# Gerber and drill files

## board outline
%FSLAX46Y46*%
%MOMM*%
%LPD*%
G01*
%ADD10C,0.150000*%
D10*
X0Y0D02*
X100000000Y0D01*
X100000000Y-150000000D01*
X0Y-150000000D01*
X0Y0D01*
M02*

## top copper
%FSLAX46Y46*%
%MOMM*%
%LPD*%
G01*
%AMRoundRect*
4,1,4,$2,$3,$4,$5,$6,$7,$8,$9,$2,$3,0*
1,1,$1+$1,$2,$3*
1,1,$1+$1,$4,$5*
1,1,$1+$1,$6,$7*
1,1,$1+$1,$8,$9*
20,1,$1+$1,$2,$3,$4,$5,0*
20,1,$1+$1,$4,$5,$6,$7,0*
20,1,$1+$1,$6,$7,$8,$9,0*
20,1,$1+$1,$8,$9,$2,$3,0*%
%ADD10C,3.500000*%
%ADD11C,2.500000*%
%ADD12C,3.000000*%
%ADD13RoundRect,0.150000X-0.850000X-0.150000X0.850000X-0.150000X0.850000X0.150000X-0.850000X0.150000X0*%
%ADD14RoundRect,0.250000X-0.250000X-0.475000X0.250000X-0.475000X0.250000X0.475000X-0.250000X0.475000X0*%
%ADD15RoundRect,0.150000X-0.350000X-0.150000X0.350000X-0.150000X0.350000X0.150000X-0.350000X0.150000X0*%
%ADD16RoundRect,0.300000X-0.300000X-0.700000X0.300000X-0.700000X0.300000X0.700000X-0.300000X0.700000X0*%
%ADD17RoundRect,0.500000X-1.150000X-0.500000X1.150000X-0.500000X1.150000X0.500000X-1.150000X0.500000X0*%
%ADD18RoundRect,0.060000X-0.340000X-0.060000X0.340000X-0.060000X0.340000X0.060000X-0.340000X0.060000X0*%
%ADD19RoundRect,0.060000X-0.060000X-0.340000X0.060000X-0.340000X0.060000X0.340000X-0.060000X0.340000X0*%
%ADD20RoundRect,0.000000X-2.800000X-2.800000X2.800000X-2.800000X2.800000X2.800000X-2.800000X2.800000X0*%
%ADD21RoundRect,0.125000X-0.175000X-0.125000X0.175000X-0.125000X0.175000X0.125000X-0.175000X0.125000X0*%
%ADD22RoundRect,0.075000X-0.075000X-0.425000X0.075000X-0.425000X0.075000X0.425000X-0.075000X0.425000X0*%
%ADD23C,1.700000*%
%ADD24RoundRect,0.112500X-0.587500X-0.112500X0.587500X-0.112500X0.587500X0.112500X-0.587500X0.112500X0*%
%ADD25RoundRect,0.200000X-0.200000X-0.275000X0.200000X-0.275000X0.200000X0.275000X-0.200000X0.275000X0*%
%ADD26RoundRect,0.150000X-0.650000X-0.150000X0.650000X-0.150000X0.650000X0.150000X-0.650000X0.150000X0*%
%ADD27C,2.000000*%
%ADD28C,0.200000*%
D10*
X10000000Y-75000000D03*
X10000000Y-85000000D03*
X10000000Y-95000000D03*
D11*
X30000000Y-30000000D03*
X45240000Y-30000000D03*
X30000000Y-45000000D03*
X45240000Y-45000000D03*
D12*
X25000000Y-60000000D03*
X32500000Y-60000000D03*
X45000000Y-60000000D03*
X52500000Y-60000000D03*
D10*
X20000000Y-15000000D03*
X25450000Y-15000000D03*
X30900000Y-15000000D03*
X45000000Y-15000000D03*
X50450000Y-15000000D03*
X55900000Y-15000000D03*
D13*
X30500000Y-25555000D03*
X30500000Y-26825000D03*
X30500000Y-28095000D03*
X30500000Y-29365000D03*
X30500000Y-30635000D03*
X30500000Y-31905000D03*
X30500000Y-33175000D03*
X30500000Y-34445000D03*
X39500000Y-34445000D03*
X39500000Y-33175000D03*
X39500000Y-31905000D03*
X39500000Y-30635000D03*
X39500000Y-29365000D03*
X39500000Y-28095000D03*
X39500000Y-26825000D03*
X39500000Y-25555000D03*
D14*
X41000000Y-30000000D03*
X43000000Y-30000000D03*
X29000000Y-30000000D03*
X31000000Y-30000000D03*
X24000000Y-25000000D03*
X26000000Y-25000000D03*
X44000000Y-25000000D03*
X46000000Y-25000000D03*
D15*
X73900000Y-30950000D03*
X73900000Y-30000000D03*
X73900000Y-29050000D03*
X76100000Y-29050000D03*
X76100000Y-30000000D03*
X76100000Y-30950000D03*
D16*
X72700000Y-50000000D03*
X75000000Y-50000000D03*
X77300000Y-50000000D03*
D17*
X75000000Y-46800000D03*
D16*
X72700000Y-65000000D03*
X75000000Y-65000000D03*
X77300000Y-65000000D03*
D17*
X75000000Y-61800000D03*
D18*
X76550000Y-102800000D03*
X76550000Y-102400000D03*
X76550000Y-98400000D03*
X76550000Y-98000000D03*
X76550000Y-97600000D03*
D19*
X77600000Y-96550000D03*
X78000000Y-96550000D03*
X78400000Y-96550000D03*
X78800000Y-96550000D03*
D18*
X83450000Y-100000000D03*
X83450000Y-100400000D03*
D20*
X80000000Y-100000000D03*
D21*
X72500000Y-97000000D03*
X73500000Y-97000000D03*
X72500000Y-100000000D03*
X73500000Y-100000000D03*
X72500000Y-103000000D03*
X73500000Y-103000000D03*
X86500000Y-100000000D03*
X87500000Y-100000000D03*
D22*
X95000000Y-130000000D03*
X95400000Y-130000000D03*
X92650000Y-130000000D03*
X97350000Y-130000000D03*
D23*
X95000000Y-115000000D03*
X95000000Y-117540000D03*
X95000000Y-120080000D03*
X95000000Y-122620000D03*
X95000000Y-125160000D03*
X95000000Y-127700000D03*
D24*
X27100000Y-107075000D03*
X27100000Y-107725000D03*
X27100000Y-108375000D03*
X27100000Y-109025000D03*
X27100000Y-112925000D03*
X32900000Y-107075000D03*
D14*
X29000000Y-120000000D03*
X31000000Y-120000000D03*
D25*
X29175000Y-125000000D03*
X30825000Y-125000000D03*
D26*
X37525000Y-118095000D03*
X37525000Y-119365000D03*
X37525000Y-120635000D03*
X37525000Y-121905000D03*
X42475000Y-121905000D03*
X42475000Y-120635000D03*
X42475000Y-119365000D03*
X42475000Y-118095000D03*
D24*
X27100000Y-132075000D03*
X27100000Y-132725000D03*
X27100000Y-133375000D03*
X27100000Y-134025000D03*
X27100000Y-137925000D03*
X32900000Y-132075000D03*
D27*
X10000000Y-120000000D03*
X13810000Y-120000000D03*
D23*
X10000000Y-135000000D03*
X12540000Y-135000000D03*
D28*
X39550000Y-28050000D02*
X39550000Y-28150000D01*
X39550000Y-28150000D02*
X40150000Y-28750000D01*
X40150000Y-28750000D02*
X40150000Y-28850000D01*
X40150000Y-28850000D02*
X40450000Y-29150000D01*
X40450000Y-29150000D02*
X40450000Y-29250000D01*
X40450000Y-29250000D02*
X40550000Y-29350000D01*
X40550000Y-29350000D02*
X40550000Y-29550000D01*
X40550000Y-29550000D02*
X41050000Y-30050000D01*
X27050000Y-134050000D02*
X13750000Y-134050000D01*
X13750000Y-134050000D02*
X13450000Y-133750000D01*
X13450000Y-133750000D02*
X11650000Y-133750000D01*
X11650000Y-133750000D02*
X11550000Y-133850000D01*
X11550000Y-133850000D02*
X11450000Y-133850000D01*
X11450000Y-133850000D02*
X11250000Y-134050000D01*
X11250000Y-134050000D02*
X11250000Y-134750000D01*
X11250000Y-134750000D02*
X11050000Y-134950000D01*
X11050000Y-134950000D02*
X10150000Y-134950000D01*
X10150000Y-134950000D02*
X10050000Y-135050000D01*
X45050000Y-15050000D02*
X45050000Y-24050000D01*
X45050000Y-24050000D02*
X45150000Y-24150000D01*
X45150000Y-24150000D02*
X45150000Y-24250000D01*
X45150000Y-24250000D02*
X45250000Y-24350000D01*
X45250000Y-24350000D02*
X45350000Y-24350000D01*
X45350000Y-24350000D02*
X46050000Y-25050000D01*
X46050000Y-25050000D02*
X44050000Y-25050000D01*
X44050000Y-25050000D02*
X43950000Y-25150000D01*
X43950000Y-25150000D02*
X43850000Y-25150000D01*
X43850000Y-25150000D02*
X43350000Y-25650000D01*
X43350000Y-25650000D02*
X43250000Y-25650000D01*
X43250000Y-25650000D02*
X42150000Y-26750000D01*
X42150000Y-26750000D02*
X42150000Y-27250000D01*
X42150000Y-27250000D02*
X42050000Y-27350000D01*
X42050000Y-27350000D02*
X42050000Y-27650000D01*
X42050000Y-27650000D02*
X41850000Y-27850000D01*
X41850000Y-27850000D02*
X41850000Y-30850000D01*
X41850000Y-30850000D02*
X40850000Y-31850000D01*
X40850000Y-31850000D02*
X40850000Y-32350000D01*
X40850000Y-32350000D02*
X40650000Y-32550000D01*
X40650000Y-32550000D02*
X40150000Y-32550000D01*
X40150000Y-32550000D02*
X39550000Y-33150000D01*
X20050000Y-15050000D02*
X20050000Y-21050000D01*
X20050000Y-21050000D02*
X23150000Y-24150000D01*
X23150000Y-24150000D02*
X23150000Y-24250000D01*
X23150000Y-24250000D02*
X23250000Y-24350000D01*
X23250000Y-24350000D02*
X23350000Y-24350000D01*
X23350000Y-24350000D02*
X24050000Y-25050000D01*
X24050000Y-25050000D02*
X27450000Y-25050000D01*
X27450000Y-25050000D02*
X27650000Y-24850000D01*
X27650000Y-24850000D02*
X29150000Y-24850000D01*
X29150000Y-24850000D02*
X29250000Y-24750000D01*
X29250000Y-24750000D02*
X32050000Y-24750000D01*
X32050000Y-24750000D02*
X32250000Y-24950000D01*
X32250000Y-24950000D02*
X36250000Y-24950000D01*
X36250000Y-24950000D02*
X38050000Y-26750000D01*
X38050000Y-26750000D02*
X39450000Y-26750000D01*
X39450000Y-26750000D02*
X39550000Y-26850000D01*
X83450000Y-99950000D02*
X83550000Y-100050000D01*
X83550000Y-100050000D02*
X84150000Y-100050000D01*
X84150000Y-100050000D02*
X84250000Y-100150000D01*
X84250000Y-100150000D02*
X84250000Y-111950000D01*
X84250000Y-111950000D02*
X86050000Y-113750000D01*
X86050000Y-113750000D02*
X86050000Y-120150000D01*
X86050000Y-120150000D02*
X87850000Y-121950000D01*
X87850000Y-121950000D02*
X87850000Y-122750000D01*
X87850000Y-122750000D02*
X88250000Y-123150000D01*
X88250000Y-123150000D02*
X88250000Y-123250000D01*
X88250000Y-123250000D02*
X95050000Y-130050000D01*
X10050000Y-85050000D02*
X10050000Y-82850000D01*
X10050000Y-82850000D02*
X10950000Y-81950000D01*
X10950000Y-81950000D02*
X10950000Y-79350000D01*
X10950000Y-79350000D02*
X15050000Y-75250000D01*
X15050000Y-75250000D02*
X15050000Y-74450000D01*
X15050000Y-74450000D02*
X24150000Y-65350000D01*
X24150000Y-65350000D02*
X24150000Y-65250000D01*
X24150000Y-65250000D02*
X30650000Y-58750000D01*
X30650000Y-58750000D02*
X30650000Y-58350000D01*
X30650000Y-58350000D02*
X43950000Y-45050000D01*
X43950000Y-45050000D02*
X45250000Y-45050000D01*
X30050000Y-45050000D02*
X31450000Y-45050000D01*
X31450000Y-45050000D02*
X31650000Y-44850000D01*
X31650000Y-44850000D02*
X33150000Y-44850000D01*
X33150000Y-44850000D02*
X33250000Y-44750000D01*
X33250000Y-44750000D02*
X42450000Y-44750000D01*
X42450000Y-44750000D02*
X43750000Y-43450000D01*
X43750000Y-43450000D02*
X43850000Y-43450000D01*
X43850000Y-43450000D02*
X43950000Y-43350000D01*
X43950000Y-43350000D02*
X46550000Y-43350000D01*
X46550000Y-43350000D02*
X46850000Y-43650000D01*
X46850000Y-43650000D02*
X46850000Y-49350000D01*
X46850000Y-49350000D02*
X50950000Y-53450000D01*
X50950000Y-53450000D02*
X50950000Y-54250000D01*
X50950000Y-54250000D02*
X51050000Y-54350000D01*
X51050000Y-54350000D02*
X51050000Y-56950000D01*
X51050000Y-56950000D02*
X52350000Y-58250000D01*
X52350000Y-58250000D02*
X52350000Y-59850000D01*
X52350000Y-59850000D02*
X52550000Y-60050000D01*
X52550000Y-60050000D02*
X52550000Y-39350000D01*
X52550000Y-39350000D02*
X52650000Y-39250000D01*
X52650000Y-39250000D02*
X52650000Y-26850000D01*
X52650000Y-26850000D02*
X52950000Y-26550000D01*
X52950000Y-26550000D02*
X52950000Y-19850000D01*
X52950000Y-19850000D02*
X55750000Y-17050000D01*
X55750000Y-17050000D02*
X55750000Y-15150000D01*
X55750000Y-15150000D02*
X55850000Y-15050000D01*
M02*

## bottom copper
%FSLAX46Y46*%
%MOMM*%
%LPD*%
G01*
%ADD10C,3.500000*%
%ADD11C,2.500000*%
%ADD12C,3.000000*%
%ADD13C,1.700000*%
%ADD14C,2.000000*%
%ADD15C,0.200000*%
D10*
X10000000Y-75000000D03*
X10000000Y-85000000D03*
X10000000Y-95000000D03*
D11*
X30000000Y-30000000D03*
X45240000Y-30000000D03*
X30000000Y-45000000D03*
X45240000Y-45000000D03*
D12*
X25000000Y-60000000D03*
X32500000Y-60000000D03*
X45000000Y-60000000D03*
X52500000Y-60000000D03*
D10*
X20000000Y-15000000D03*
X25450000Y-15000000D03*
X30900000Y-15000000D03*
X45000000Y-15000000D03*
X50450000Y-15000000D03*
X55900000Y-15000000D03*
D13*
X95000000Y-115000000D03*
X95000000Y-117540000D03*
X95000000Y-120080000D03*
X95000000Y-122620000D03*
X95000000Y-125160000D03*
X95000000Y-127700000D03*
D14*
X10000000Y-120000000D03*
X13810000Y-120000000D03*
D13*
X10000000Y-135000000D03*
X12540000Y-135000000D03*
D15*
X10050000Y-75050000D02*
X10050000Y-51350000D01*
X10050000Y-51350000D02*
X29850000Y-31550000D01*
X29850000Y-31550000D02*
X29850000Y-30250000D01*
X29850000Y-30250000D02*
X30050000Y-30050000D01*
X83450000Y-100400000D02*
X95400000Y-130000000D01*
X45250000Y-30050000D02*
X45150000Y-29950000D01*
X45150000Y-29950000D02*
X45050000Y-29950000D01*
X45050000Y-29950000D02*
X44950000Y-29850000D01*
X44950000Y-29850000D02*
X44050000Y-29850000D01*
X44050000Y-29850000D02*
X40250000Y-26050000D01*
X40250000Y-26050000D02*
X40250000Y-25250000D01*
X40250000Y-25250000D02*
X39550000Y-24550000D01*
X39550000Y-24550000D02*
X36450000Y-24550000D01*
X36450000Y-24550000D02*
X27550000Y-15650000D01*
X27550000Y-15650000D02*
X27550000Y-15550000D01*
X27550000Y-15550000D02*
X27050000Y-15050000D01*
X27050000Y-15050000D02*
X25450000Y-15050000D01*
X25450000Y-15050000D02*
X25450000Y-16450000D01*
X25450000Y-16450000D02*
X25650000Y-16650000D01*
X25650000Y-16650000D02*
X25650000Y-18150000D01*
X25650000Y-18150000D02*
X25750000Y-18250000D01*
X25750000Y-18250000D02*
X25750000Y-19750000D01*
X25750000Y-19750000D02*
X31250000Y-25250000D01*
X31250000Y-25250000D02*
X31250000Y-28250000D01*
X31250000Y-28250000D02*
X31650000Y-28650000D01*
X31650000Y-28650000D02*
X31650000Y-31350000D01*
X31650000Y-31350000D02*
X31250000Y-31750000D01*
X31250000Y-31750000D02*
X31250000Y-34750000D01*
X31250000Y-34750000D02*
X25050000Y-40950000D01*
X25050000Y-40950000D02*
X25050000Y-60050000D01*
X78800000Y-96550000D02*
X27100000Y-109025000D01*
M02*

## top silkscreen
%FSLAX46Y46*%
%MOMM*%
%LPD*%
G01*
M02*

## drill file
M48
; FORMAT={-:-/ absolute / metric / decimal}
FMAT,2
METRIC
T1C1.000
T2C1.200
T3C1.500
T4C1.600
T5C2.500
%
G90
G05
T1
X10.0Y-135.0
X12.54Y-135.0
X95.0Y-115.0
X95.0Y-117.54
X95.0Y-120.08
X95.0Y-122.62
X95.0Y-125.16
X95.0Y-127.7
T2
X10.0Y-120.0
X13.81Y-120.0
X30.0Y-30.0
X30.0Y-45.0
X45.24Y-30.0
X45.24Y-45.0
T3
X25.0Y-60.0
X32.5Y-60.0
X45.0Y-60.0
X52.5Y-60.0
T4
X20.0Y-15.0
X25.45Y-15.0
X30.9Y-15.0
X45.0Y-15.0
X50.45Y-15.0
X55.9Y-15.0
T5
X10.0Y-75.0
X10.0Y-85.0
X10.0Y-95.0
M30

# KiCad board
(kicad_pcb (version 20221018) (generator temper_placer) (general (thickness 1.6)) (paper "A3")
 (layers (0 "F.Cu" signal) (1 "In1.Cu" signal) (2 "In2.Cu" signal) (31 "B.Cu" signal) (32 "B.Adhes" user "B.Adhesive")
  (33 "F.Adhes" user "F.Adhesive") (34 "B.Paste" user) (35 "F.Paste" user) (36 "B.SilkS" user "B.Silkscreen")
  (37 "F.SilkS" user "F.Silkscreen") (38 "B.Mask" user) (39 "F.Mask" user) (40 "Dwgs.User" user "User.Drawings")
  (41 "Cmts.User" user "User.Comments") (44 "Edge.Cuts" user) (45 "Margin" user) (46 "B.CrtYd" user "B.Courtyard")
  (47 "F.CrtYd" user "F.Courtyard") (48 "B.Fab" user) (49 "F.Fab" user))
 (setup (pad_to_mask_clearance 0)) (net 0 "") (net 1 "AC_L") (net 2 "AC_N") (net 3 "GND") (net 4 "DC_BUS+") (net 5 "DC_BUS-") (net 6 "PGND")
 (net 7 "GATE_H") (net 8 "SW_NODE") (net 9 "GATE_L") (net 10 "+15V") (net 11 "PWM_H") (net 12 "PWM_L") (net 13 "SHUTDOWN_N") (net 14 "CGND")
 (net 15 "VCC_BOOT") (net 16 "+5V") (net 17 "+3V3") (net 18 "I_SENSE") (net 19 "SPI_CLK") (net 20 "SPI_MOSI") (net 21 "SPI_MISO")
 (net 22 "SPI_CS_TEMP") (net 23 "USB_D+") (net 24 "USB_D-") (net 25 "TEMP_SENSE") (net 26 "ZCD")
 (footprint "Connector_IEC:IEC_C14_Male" (layer "F.Cu") (at 10 75) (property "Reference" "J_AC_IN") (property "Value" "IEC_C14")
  (pad "1" thru_hole circle (at 0 0) (size 3.5 3.5) (drill 2.5) (layers *.Cu *.Mask) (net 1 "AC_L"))
  (pad "2" thru_hole circle (at 0 10) (size 3.5 3.5) (drill 2.5) (layers *.Cu *.Mask) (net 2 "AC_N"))
  (pad "3" thru_hole circle (at 0 20) (size 3.5 3.5) (drill 2.5) (layers *.Cu *.Mask) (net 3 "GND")))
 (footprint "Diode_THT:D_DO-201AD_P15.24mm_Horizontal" (layer "F.Cu") (at 30 30) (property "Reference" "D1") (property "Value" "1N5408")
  (pad "1" thru_hole circle (at 0 0) (size 2.5 2.5) (drill 1.2) (layers *.Cu *.Mask) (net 1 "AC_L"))
  (pad "2" thru_hole circle (at 15.24 0) (size 2.5 2.5) (drill 1.2) (layers *.Cu *.Mask) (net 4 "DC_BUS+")))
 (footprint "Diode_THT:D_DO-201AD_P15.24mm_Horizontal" (layer "F.Cu") (at 30 45) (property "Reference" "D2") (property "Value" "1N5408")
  (pad "1" thru_hole circle (at 0 0) (size 2.5 2.5) (drill 1.2) (layers *.Cu *.Mask) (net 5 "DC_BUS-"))
  (pad "2" thru_hole circle (at 15.24 0) (size 2.5 2.5) (drill 1.2) (layers *.Cu *.Mask) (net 2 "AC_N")))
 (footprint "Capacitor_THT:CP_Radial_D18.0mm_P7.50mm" (layer "F.Cu") (at 25 60) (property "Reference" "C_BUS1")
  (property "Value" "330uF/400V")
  (pad "1" thru_hole circle (at 0 0) (size 3 3) (drill 1.5) (layers *.Cu *.Mask) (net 4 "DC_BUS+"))
  (pad "2" thru_hole circle (at 7.5 0) (size 3 3) (drill 1.5) (layers *.Cu *.Mask) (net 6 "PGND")))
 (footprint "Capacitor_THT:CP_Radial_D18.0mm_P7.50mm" (layer "F.Cu") (at 45 60) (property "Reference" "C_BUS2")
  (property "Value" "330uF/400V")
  (pad "1" thru_hole circle (at 0 0) (size 3 3) (drill 1.5) (layers *.Cu *.Mask) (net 6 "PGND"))
  (pad "2" thru_hole circle (at 7.5 0) (size 3 3) (drill 1.5) (layers *.Cu *.Mask) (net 5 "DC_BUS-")))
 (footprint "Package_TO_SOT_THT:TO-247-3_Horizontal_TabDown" (layer "F.Cu") (at 20 15) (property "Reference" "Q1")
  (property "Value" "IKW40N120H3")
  (pad "1" thru_hole circle (at 0 0) (size 3.5 3.5) (drill 1.6) (layers *.Cu *.Mask) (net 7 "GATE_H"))
  (pad "2" thru_hole circle (at 5.45 0) (size 3.5 3.5) (drill 1.6) (layers *.Cu *.Mask) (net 4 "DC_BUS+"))
  (pad "3" thru_hole circle (at 10.9 0) (size 3.5 3.5) (drill 1.6) (layers *.Cu *.Mask) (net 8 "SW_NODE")))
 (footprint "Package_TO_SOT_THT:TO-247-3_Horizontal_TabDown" (layer "F.Cu") (at 45 15) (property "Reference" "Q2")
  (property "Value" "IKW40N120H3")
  (pad "1" thru_hole circle (at 0 0) (size 3.5 3.5) (drill 1.6) (layers *.Cu *.Mask) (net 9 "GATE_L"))
  (pad "2" thru_hole circle (at 5.45 0) (size 3.5 3.5) (drill 1.6) (layers *.Cu *.Mask) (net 8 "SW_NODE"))
  (pad "3" thru_hole circle (at 10.9 0) (size 3.5 3.5) (drill 1.6) (layers *.Cu *.Mask) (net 5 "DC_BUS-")))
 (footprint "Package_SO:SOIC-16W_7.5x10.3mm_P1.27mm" (layer "F.Cu") (at 35 30) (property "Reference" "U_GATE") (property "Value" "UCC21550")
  (pad "1" smd roundrect (at -4.5 -4.445) (size 2 0.6) (layers "F.Cu" "F.Paste" "F.Mask") (roundrect_rratio 0.25) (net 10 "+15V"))
  (pad "2" smd roundrect (at -4.5 -3.175) (size 2 0.6) (layers "F.Cu" "F.Paste" "F.Mask") (roundrect_rratio 0.25) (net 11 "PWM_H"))
  (pad "3" smd roundrect (at -4.5 -1.905) (size 2 0.6) (layers "F.Cu" "F.Paste" "F.Mask") (roundrect_rratio 0.25) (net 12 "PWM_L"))
  (pad "4" smd roundrect (at -4.5 -0.635) (size 2 0.6) (layers "F.Cu" "F.Paste" "F.Mask") (roundrect_rratio 0.25) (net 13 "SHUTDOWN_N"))
  (pad "5" smd roundrect (at -4.5 0.635) (size 2 0.6) (layers "F.Cu" "F.Paste" "F.Mask") (roundrect_rratio 0.25) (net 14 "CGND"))
  (pad "6" smd roundrect (at -4.5 1.905) (size 2 0.6) (layers "F.Cu" "F.Paste" "F.Mask") (roundrect_rratio 0.25) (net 14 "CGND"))
  (pad "7" smd roundrect (at -4.5 3.175) (size 2 0.6) (layers "F.Cu" "F.Paste" "F.Mask") (roundrect_rratio 0.25) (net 14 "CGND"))
  (pad "8" smd roundrect (at -4.5 4.445) (size 2 0.6) (layers "F.Cu" "F.Paste" "F.Mask") (roundrect_rratio 0.25) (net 14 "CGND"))
  (pad "9" smd roundrect (at 4.5 4.445) (size 2 0.6) (layers "F.Cu" "F.Paste" "F.Mask") (roundrect_rratio 0.25) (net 8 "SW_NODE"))
  (pad "10" smd roundrect (at 4.5 3.175) (size 2 0.6) (layers "F.Cu" "F.Paste" "F.Mask") (roundrect_rratio 0.25) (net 9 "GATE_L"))
  (pad "11" smd roundrect (at 4.5 1.905) (size 2 0.6) (layers "F.Cu" "F.Paste" "F.Mask") (roundrect_rratio 0.25) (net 10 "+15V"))
  (pad "12" smd roundrect (at 4.5 0.635) (size 2 0.6) (layers "F.Cu" "F.Paste" "F.Mask") (roundrect_rratio 0.25) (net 6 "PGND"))
  (pad "13" smd roundrect (at 4.5 -0.635) (size 2 0.6) (layers "F.Cu" "F.Paste" "F.Mask") (roundrect_rratio 0.25) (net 6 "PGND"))
  (pad "14" smd roundrect (at 4.5 -1.905) (size 2 0.6) (layers "F.Cu" "F.Paste" "F.Mask") (roundrect_rratio 0.25) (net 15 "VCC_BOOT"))
  (pad "15" smd roundrect (at 4.5 -3.175) (size 2 0.6) (layers "F.Cu" "F.Paste" "F.Mask") (roundrect_rratio 0.25) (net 7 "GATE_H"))
  (pad "16" smd roundrect (at 4.5 -4.445) (size 2 0.6) (layers "F.Cu" "F.Paste" "F.Mask") (roundrect_rratio 0.25) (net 8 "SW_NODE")))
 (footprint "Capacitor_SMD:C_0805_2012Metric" (layer "F.Cu") (at 42 30) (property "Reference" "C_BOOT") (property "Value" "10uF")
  (pad "1" smd roundrect (at -1 0) (size 1 1.45) (layers "F.Cu" "F.Paste" "F.Mask") (roundrect_rratio 0.25) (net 15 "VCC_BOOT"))
  (pad "2" smd roundrect (at 1 0) (size 1 1.45) (layers "F.Cu" "F.Paste" "F.Mask") (roundrect_rratio 0.25) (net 8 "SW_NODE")))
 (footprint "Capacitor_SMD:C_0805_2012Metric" (layer "F.Cu") (at 30 30) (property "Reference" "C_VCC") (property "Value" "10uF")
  (pad "1" smd roundrect (at -1 0) (size 1 1.45) (layers "F.Cu" "F.Paste" "F.Mask") (roundrect_rratio 0.25) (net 10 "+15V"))
  (pad "2" smd roundrect (at 1 0) (size 1 1.45) (layers "F.Cu" "F.Paste" "F.Mask") (roundrect_rratio 0.25) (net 14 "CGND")))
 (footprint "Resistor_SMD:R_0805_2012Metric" (layer "F.Cu") (at 25 25) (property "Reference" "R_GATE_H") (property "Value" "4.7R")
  (pad "1" smd roundrect (at -1 0) (size 1 1.45) (layers "F.Cu" "F.Paste" "F.Mask") (roundrect_rratio 0.25) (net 7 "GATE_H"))
  (pad "2" smd roundrect (at 1 0) (size 1 1.45) (layers "F.Cu" "F.Paste" "F.Mask") (roundrect_rratio 0.25) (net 7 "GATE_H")))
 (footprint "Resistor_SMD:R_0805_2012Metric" (layer "F.Cu") (at 45 25) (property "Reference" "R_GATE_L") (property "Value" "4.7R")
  (pad "1" smd roundrect (at -1 0) (size 1 1.45) (layers "F.Cu" "F.Paste" "F.Mask") (roundrect_rratio 0.25) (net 9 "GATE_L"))
  (pad "2" smd roundrect (at 1 0) (size 1 1.45) (layers "F.Cu" "F.Paste" "F.Mask") (roundrect_rratio 0.25) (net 9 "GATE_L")))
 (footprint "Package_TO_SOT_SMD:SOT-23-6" (layer "F.Cu") (at 75 30) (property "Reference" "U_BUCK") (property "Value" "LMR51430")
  (pad "1" smd roundrect (at -1.1 0.95) (size 1 0.6) (layers "F.Cu" "F.Paste" "F.Mask") (roundrect_rratio 0.25) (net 3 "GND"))
  (pad "2" smd roundrect (at -1.1 0) (size 1 0.6) (layers "F.Cu" "F.Paste" "F.Mask") (roundrect_rratio 0.25) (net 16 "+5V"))
  (pad "3" smd roundrect (at -1.1 -0.95) (size 1 0.6) (layers "F.Cu" "F.Paste" "F.Mask") (roundrect_rratio 0.25) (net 10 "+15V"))
  (pad "4" smd roundrect (at 1.1 -0.95) (size 1 0.6) (layers "F.Cu" "F.Paste" "F.Mask") (roundrect_rratio 0.25) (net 16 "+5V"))
  (pad "5" smd roundrect (at 1.1 0) (size 1 0.6) (layers "F.Cu" "F.Paste" "F.Mask") (roundrect_rratio 0.25) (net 3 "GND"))
  (pad "6" smd roundrect (at 1.1 0.95) (size 1 0.6) (layers "F.Cu" "F.Paste" "F.Mask") (roundrect_rratio 0.25) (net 3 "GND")))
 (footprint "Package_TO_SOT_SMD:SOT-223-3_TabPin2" (layer "F.Cu") (at 75 50) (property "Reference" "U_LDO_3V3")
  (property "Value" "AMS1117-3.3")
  (pad "1" smd roundrect (at -2.3 0) (size 1.2 2) (layers "F.Cu" "F.Paste" "F.Mask") (roundrect_rratio 0.25) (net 3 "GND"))
  (pad "2" smd roundrect (at 0 0) (size 1.2 2) (layers "F.Cu" "F.Paste" "F.Mask") (roundrect_rratio 0.25) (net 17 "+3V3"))
  (pad "3" smd roundrect (at 2.3 0) (size 1.2 2) (layers "F.Cu" "F.Paste" "F.Mask") (roundrect_rratio 0.25) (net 16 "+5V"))
  (pad "4" smd roundrect (at 0 -3.2) (size 3.3 2) (layers "F.Cu" "F.Paste" "F.Mask") (roundrect_rratio 0.25) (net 17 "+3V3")))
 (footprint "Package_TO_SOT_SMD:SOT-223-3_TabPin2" (layer "F.Cu") (at 75 65) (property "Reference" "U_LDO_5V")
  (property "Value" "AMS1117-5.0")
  (pad "1" smd roundrect (at -2.3 0) (size 1.2 2) (layers "F.Cu" "F.Paste" "F.Mask") (roundrect_rratio 0.25) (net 3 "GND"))
  (pad "2" smd roundrect (at 0 0) (size 1.2 2) (layers "F.Cu" "F.Paste" "F.Mask") (roundrect_rratio 0.25) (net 16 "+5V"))
  (pad "3" smd roundrect (at 2.3 0) (size 1.2 2) (layers "F.Cu" "F.Paste" "F.Mask") (roundrect_rratio 0.25) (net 10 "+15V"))
  (pad "4" smd roundrect (at 0 -3.2) (size 3.3 2) (layers "F.Cu" "F.Paste" "F.Mask") (roundrect_rratio 0.25) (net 16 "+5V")))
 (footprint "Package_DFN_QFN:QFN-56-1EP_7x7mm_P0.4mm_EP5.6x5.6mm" (layer "F.Cu") (at 80 100) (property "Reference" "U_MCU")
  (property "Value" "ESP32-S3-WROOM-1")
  (pad "1" smd roundrect (at -3.45 2.8) (size 0.8 0.24) (layers "F.Cu" "F.Paste" "F.Mask") (roundrect_rratio 0.25) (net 17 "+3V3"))
  (pad "2" smd roundrect (at -3.45 2.4) (size 0.8 0.24) (layers "F.Cu" "F.Paste" "F.Mask") (roundrect_rratio 0.25) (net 3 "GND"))
  (pad "13" smd roundrect (at -3.45 -1.6) (size 0.8 0.24) (layers "F.Cu" "F.Paste" "F.Mask") (roundrect_rratio 0.25) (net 11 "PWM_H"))
  (pad "14" smd roundrect (at -3.45 -2) (size 0.8 0.24) (layers "F.Cu" "F.Paste" "F.Mask") (roundrect_rratio 0.25) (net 12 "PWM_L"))
  (pad "15" smd roundrect (at -3.45 -2.4) (size 0.8 0.24) (layers "F.Cu" "F.Paste" "F.Mask") (roundrect_rratio 0.25) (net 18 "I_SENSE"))
  (pad "20" smd roundrect (at -2.4 -3.45) (size 0.24 0.8) (layers "F.Cu" "F.Paste" "F.Mask") (roundrect_rratio 0.25) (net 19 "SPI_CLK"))
  (pad "21" smd roundrect (at -2 -3.45) (size 0.24 0.8) (layers "F.Cu" "F.Paste" "F.Mask") (roundrect_rratio 0.25) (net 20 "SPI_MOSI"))
  (pad "22" smd roundrect (at -1.6 -3.45) (size 0.24 0.8) (layers "F.Cu" "F.Paste" "F.Mask") (roundrect_rratio 0.25) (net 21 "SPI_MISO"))
  (pad "23" smd roundrect (at -1.2 -3.45) (size 0.24 0.8) (layers "F.Cu" "F.Paste" "F.Mask") (roundrect_rratio 0.25) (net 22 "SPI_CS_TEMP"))
  (pad "40" smd roundrect (at 3.45 0) (size 0.8 0.24) (layers "F.Cu" "F.Paste" "F.Mask") (roundrect_rratio 0.25) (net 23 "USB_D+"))
  (pad "41" smd roundrect (at 3.45 0.4) (size 0.8 0.24) (layers "F.Cu" "F.Paste" "F.Mask") (roundrect_rratio 0.25) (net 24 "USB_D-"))
  (pad "57" smd roundrect (at 0 0) (size 5.6 5.6) (layers "F.Cu" "F.Paste" "F.Mask") (roundrect_rratio 0) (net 3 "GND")))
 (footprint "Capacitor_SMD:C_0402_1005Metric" (layer "F.Cu") (at 73 97) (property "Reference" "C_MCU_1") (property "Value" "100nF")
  (pad "1" smd roundrect (at -0.5 0) (size 0.6 0.5) (layers "F.Cu" "F.Paste" "F.Mask") (roundrect_rratio 0.25) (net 17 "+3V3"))
  (pad "2" smd roundrect (at 0.5 0) (size 0.6 0.5) (layers "F.Cu" "F.Paste" "F.Mask") (roundrect_rratio 0.25) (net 3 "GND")))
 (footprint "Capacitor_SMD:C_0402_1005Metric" (layer "F.Cu") (at 73 100) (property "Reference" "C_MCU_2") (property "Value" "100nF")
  (pad "1" smd roundrect (at -0.5 0) (size 0.6 0.5) (layers "F.Cu" "F.Paste" "F.Mask") (roundrect_rratio 0.25) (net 17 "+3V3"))
  (pad "2" smd roundrect (at 0.5 0) (size 0.6 0.5) (layers "F.Cu" "F.Paste" "F.Mask") (roundrect_rratio 0.25) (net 3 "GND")))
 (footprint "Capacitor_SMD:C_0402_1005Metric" (layer "F.Cu") (at 73 103) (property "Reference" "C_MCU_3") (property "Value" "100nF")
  (pad "1" smd roundrect (at -0.5 0) (size 0.6 0.5) (layers "F.Cu" "F.Paste" "F.Mask") (roundrect_rratio 0.25) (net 17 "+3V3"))
  (pad "2" smd roundrect (at 0.5 0) (size 0.6 0.5) (layers "F.Cu" "F.Paste" "F.Mask") (roundrect_rratio 0.25) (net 3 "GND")))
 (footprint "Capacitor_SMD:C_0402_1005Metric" (layer "F.Cu") (at 87 100) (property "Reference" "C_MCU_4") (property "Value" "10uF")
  (pad "1" smd roundrect (at -0.5 0) (size 0.6 0.5) (layers "F.Cu" "F.Paste" "F.Mask") (roundrect_rratio 0.25) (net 17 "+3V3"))
  (pad "2" smd roundrect (at 0.5 0) (size 0.6 0.5) (layers "F.Cu" "F.Paste" "F.Mask") (roundrect_rratio 0.25) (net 3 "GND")))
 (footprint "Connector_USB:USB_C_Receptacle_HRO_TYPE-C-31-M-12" (layer "F.Cu") (at 95 130) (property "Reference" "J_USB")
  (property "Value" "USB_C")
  (pad "A6" smd roundrect (at 0 0) (size 0.3 1) (layers "F.Cu" "F.Paste" "F.Mask") (roundrect_rratio 0.25) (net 23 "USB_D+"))
  (pad "B6" smd roundrect (at 0.4 0) (size 0.3 1) (layers "F.Cu" "F.Paste" "F.Mask") (roundrect_rratio 0.25) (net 24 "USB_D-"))
  (pad "A1" smd roundrect (at -2.35 0) (size 0.3 1) (layers "F.Cu" "F.Paste" "F.Mask") (roundrect_rratio 0.25) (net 3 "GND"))
  (pad "A12" smd roundrect (at 2.35 0) (size 0.3 1) (layers "F.Cu" "F.Paste" "F.Mask") (roundrect_rratio 0.25) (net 3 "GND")))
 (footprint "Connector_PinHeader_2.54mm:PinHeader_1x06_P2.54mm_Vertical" (layer "F.Cu") (at 95 115) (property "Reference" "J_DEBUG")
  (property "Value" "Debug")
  (pad "1" thru_hole circle (at 0 0) (size 1.7 1.7) (drill 1) (layers *.Cu *.Mask) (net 3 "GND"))
  (pad "2" thru_hole circle (at 0 2.54) (size 1.7 1.7) (drill 1) (layers *.Cu *.Mask) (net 17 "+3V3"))
  (pad "3" thru_hole circle (at 0 5.08) (size 1.7 1.7) (drill 1) (layers *.Cu *.Mask) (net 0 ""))
  (pad "4" thru_hole circle (at 0 7.62) (size 1.7 1.7) (drill 1) (layers *.Cu *.Mask) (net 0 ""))
  (pad "5" thru_hole circle (at 0 10.16) (size 1.7 1.7) (drill 1) (layers *.Cu *.Mask) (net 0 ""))
  (pad "6" thru_hole circle (at 0 12.7) (size 1.7 1.7) (drill 1) (layers *.Cu *.Mask) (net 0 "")))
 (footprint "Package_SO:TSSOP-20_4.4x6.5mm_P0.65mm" (layer "F.Cu") (at 30 110) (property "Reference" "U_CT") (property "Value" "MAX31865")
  (pad "1" smd roundrect (at -2.9 -2.925) (size 1.4 0.45) (layers "F.Cu" "F.Paste" "F.Mask") (roundrect_rratio 0.25) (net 19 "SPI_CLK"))
  (pad "2" smd roundrect (at -2.9 -2.275) (size 1.4 0.45) (layers "F.Cu" "F.Paste" "F.Mask") (roundrect_rratio 0.25) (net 20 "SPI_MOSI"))
  (pad "3" smd roundrect (at -2.9 -1.625) (size 1.4 0.45) (layers "F.Cu" "F.Paste" "F.Mask") (roundrect_rratio 0.25) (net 21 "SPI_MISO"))
  (pad "4" smd roundrect (at -2.9 -0.975) (size 1.4 0.45) (layers "F.Cu" "F.Paste" "F.Mask") (roundrect_rratio 0.25) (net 22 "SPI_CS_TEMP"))
  (pad "10" smd roundrect (at -2.9 2.925) (size 1.4 0.45) (layers "F.Cu" "F.Paste" "F.Mask") (roundrect_rratio 0.25) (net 3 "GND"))
  (pad "20" smd roundrect (at 2.9 -2.925) (size 1.4 0.45) (layers "F.Cu" "F.Paste" "F.Mask") (roundrect_rratio 0.25) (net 17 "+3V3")))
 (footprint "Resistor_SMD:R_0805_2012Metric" (layer "F.Cu") (at 30 120) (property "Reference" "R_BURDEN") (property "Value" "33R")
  (pad "1" smd roundrect (at -1 0) (size 1 1.45) (layers "F.Cu" "F.Paste" "F.Mask") (roundrect_rratio 0.25) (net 18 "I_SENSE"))
  (pad "2" smd roundrect (at 1 0) (size 1 1.45) (layers "F.Cu" "F.Paste" "F.Mask") (roundrect_rratio 0.25) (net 3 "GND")))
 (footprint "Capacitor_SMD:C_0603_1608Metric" (layer "F.Cu") (at 30 125) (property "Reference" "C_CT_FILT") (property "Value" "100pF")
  (pad "1" smd roundrect (at -0.825 0) (size 0.8 0.95) (layers "F.Cu" "F.Paste" "F.Mask") (roundrect_rratio 0.25) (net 18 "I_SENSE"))
  (pad "2" smd roundrect (at 0.825 0) (size 0.8 0.95) (layers "F.Cu" "F.Paste" "F.Mask") (roundrect_rratio 0.25) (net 3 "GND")))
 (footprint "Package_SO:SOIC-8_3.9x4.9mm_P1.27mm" (layer "F.Cu") (at 40 120) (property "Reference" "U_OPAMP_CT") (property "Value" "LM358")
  (pad "1" smd roundrect (at -2.475 -1.905) (size 1.6 0.6) (layers "F.Cu" "F.Paste" "F.Mask") (roundrect_rratio 0.25) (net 18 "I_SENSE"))
  (pad "2" smd roundrect (at -2.475 -0.635) (size 1.6 0.6) (layers "F.Cu" "F.Paste" "F.Mask") (roundrect_rratio 0.25) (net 18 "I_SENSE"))
  (pad "3" smd roundrect (at -2.475 0.635) (size 1.6 0.6) (layers "F.Cu" "F.Paste" "F.Mask") (roundrect_rratio 0.25) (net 18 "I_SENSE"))
  (pad "4" smd roundrect (at -2.475 1.905) (size 1.6 0.6) (layers "F.Cu" "F.Paste" "F.Mask") (roundrect_rratio 0.25) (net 3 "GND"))
  (pad "5" smd roundrect (at 2.475 1.905) (size 1.6 0.6) (layers "F.Cu" "F.Paste" "F.Mask") (roundrect_rratio 0.25) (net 18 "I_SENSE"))
  (pad "6" smd roundrect (at 2.475 0.635) (size 1.6 0.6) (layers "F.Cu" "F.Paste" "F.Mask") (roundrect_rratio 0.25) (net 18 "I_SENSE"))
  (pad "7" smd roundrect (at 2.475 -0.635) (size 1.6 0.6) (layers "F.Cu" "F.Paste" "F.Mask") (roundrect_rratio 0.25) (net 16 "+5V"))
  (pad "8" smd roundrect (at 2.475 -1.905) (size 1.6 0.6) (layers "F.Cu" "F.Paste" "F.Mask") (roundrect_rratio 0.25) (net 16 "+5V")))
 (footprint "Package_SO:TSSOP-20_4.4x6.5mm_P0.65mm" (layer "F.Cu") (at 30 135) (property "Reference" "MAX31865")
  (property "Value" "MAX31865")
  (pad "1" smd roundrect (at -2.9 -2.925) (size 1.4 0.45) (layers "F.Cu" "F.Paste" "F.Mask") (roundrect_rratio 0.25) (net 19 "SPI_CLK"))
  (pad "2" smd roundrect (at -2.9 -2.275) (size 1.4 0.45) (layers "F.Cu" "F.Paste" "F.Mask") (roundrect_rratio 0.25) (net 20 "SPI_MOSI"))
  (pad "3" smd roundrect (at -2.9 -1.625) (size 1.4 0.45) (layers "F.Cu" "F.Paste" "F.Mask") (roundrect_rratio 0.25) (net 21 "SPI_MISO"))
  (pad "4" smd roundrect (at -2.9 -0.975) (size 1.4 0.45) (layers "F.Cu" "F.Paste" "F.Mask") (roundrect_rratio 0.25) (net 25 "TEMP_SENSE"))
  (pad "10" smd roundrect (at -2.9 2.925) (size 1.4 0.45) (layers "F.Cu" "F.Paste" "F.Mask") (roundrect_rratio 0.25) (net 3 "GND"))
  (pad "20" smd roundrect (at 2.9 -2.925) (size 1.4 0.45) (layers "F.Cu" "F.Paste" "F.Mask") (roundrect_rratio 0.25) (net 17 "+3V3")))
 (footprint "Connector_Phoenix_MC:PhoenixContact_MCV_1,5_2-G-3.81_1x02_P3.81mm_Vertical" (layer "F.Cu") (at 10 120)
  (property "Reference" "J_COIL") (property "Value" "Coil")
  (pad "1" thru_hole circle (at 0 0) (size 2 2) (drill 1.2) (layers *.Cu *.Mask) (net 8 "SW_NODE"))
  (pad "2" thru_hole circle (at 3.81 0) (size 2 2) (drill 1.2) (layers *.Cu *.Mask) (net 3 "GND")))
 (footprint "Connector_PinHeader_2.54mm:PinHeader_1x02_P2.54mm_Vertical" (layer "F.Cu") (at 10 135) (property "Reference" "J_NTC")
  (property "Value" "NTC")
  (pad "1" thru_hole circle (at 0 0) (size 1.7 1.7) (drill 1) (layers *.Cu *.Mask) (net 25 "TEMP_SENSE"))
  (pad "2" thru_hole circle (at 2.54 0) (size 1.7 1.7) (drill 1) (layers *.Cu *.Mask) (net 3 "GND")))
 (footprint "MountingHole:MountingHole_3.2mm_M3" (layer "F.Cu") (at 5 5) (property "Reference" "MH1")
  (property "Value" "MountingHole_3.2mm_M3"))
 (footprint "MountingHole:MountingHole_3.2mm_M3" (layer "F.Cu") (at 95 5) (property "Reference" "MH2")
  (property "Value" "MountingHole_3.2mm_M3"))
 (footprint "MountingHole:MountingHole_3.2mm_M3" (layer "F.Cu") (at 5 145) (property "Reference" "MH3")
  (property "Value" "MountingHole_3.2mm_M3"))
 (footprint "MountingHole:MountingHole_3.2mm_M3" (layer "F.Cu") (at 95 145) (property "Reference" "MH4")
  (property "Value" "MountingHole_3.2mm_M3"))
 (gr_rect (start 0 0) (end 100 150) (layer "Edge.Cuts") (width 0.15))
 (segment (start 39.550000000000004 28.05) (end 39.550000000000004 28.150000000000002) (width 0.2) (layer "F.Cu") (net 15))
 (segment (start 39.550000000000004 28.150000000000002) (end 40.150000000000006 28.75) (width 0.2) (layer "F.Cu") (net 15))
 (segment (start 40.150000000000006 28.75) (end 40.150000000000006 28.85) (width 0.2) (layer "F.Cu") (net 15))
 (segment (start 40.150000000000006 28.85) (end 40.45 29.150000000000002) (width 0.2) (layer "F.Cu") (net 15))
 (segment (start 40.45 29.150000000000002) (end 40.45 29.25) (width 0.2) (layer "F.Cu") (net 15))
 (segment (start 40.45 29.25) (end 40.550000000000004 29.35) (width 0.2) (layer "F.Cu") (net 15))
 (segment (start 40.550000000000004 29.35) (end 40.550000000000004 29.55) (width 0.2) (layer "F.Cu") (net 15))
 (segment (start 40.550000000000004 29.55) (end 41.050000000000004 30.050000000000004) (width 0.2) (layer "F.Cu") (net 15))
 (segment (start 10.05 75.05000000000001) (end 10.05 51.35) (width 0.2) (layer "B.Cu") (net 1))
 (segment (start 10.05 51.35) (end 29.85 31.550000000000004) (width 0.2) (layer "B.Cu") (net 1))
 (segment (start 29.85 31.550000000000004) (end 29.85 30.25) (width 0.2) (layer "B.Cu") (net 1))
 (segment (start 29.85 30.25) (end 30.050000000000004 30.050000000000004) (width 0.2) (layer "B.Cu") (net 1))
 (segment (start 27.05 134.05) (end 13.75 134.05) (width 0.2) (layer "F.Cu") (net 25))
 (segment (start 13.75 134.05) (end 13.450000000000001 133.75) (width 0.2) (layer "F.Cu") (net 25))
 (segment (start 13.450000000000001 133.75) (end 11.65 133.75) (width 0.2) (layer "F.Cu") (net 25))
 (segment (start 11.65 133.75) (end 11.55 133.85) (width 0.2) (layer "F.Cu") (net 25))
 (segment (start 11.55 133.85) (end 11.450000000000001 133.85) (width 0.2) (layer "F.Cu") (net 25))
 (segment (start 11.450000000000001 133.85) (end 11.25 134.05) (width 0.2) (layer "F.Cu") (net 25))
 (segment (start 11.25 134.05) (end 11.25 134.75) (width 0.2) (layer "F.Cu") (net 25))
 (segment (start 11.25 134.75) (end 11.05 134.95000000000002) (width 0.2) (layer "F.Cu") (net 25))
 (segment (start 11.05 134.95000000000002) (end 10.15 134.95000000000002) (width 0.2) (layer "F.Cu") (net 25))
 (segment (start 10.15 134.95000000000002) (end 10.05 135.05) (width 0.2) (layer "F.Cu") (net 25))
 (segment (start 45.050000000000004 15.05) (end 45.050000000000004 24.05) (width 0.2) (layer "F.Cu") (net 9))
 (segment (start 45.050000000000004 24.05) (end 45.150000000000006 24.150000000000002) (width 0.2) (layer "F.Cu") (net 9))
 (segment (start 45.150000000000006 24.150000000000002) (end 45.150000000000006 24.25) (width 0.2) (layer "F.Cu") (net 9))
 (segment (start 45.150000000000006 24.25) (end 45.25 24.35) (width 0.2) (layer "F.Cu") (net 9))
 (segment (start 45.25 24.35) (end 45.35 24.35) (width 0.2) (layer "F.Cu") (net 9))
 (segment (start 45.35 24.35) (end 46.050000000000004 25.05) (width 0.2) (layer "F.Cu") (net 9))
 (segment (start 46.050000000000004 25.05) (end 44.050000000000004 25.05) (width 0.2) (layer "F.Cu") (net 9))
 (segment (start 44.050000000000004 25.05) (end 43.95 25.150000000000002) (width 0.2) (layer "F.Cu") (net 9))
 (segment (start 43.95 25.150000000000002) (end 43.85 25.150000000000002) (width 0.2) (layer "F.Cu") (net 9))
 (segment (start 43.85 25.150000000000002) (end 43.35 25.650000000000002) (width 0.2) (layer "F.Cu") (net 9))
 (segment (start 43.35 25.650000000000002) (end 43.25 25.650000000000002) (width 0.2) (layer "F.Cu") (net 9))
 (segment (start 43.25 25.650000000000002) (end 42.150000000000006 26.75) (width 0.2) (layer "F.Cu") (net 9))
 (segment (start 42.150000000000006 26.75) (end 42.150000000000006 27.25) (width 0.2) (layer "F.Cu") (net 9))
 (segment (start 42.150000000000006 27.25) (end 42.050000000000004 27.35) (width 0.2) (layer "F.Cu") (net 9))
 (segment (start 42.050000000000004 27.35) (end 42.050000000000004 27.650000000000002) (width 0.2) (layer "F.Cu") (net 9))
 (segment (start 42.050000000000004 27.650000000000002) (end 41.85 27.85) (width 0.2) (layer "F.Cu") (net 9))
 (segment (start 41.85 27.85) (end 41.85 30.85) (width 0.2) (layer "F.Cu") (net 9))
 (segment (start 41.85 30.85) (end 40.85 31.85) (width 0.2) (layer "F.Cu") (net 9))
 (segment (start 40.85 31.85) (end 40.85 32.35) (width 0.2) (layer "F.Cu") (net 9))
 (segment (start 40.85 32.35) (end 40.650000000000006 32.550000000000004) (width 0.2) (layer "F.Cu") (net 9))
 (segment (start 40.650000000000006 32.550000000000004) (end 40.150000000000006 32.550000000000004) (width 0.2) (layer "F.Cu") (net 9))
 (segment (start 40.150000000000006 32.550000000000004) (end 39.550000000000004 33.15) (width 0.2) (layer "F.Cu") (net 9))
 (segment (start 20.05 15.05) (end 20.05 21.05) (width 0.2) (layer "F.Cu") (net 7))
 (segment (start 20.05 21.05) (end 23.150000000000002 24.150000000000002) (width 0.2) (layer "F.Cu") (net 7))
 (segment (start 23.150000000000002 24.150000000000002) (end 23.150000000000002 24.25) (width 0.2) (layer "F.Cu") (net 7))
 (segment (start 23.150000000000002 24.25) (end 23.25 24.35) (width 0.2) (layer "F.Cu") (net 7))
 (segment (start 23.25 24.35) (end 23.35 24.35) (width 0.2) (layer "F.Cu") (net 7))
 (segment (start 23.35 24.35) (end 24.05 25.05) (width 0.2) (layer "F.Cu") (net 7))
 (segment (start 24.05 25.05) (end 27.450000000000003 25.05) (width 0.2) (layer "F.Cu") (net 7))
 (segment (start 27.450000000000003 25.05) (end 27.650000000000002 24.85) (width 0.2) (layer "F.Cu") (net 7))
 (segment (start 27.650000000000002 24.85) (end 29.150000000000002 24.85) (width 0.2) (layer "F.Cu") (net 7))
 (segment (start 29.150000000000002 24.85) (end 29.25 24.75) (width 0.2) (layer "F.Cu") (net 7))
 (segment (start 29.25 24.75) (end 32.050000000000004 24.75) (width 0.2) (layer "F.Cu") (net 7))
 (segment (start 32.050000000000004 24.75) (end 32.25 24.950000000000003) (width 0.2) (layer "F.Cu") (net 7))
 (segment (start 32.25 24.950000000000003) (end 36.25 24.950000000000003) (width 0.2) (layer "F.Cu") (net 7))
 (segment (start 36.25 24.950000000000003) (end 38.050000000000004 26.75) (width 0.2) (layer "F.Cu") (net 7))
 (segment (start 38.050000000000004 26.75) (end 39.45 26.75) (width 0.2) (layer "F.Cu") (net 7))
 (segment (start 39.45 26.75) (end 39.550000000000004 26.85) (width 0.2) (layer "F.Cu") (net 7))
 (segment (start 83.45000004768372 100.40000002384186) (end 95.40000000596046 130.0) (width 0.2) (layer "B.Cu") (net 24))
 (segment (start 83.45 99.95) (end 83.55000000000001 100.05000000000001) (width 0.2) (layer "F.Cu") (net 23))
 (segment (start 83.55000000000001 100.05000000000001) (end 84.15 100.05000000000001) (width 0.2) (layer "F.Cu") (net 23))
 (segment (start 84.15 100.05000000000001) (end 84.25 100.15) (width 0.2) (layer "F.Cu") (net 23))
 (segment (start 84.25 100.15) (end 84.25 111.95) (width 0.2) (layer "F.Cu") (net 23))
 (segment (start 84.25 111.95) (end 86.05000000000001 113.75) (width 0.2) (layer "F.Cu") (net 23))
 (segment (start 86.05000000000001 113.75) (end 86.05000000000001 120.15) (width 0.2) (layer "F.Cu") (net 23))
 (segment (start 86.05000000000001 120.15) (end 87.85000000000001 121.95) (width 0.2) (layer "F.Cu") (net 23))
 (segment (start 87.85000000000001 121.95) (end 87.85000000000001 122.75) (width 0.2) (layer "F.Cu") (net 23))
 (segment (start 87.85000000000001 122.75) (end 88.25 123.15) (width 0.2) (layer "F.Cu") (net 23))
 (segment (start 88.25 123.15) (end 88.25 123.25) (width 0.2) (layer "F.Cu") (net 23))
 (segment (start 88.25 123.25) (end 95.05000000000001 130.05) (width 0.2) (layer "F.Cu") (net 23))
 (segment (start 10.05 85.05000000000001) (end 10.05 82.85000000000001) (width 0.2) (layer "F.Cu") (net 2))
 (segment (start 10.05 82.85000000000001) (end 10.950000000000001 81.95) (width 0.2) (layer "F.Cu") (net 2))
 (segment (start 10.950000000000001 81.95) (end 10.950000000000001 79.35000000000001) (width 0.2) (layer "F.Cu") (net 2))
 (segment (start 10.950000000000001 79.35000000000001) (end 15.05 75.25) (width 0.2) (layer "F.Cu") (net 2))
 (segment (start 15.05 75.25) (end 15.05 74.45) (width 0.2) (layer "F.Cu") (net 2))
 (segment (start 15.05 74.45) (end 24.150000000000002 65.35000000000001) (width 0.2) (layer "F.Cu") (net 2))
 (segment (start 24.150000000000002 65.35000000000001) (end 24.150000000000002 65.25) (width 0.2) (layer "F.Cu") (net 2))
 (segment (start 24.150000000000002 65.25) (end 30.65 58.75) (width 0.2) (layer "F.Cu") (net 2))
 (segment (start 30.65 58.75) (end 30.65 58.35) (width 0.2) (layer "F.Cu") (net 2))
 (segment (start 30.65 58.35) (end 43.95 45.050000000000004) (width 0.2) (layer "F.Cu") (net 2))
 (segment (start 43.95 45.050000000000004) (end 45.25 45.050000000000004) (width 0.2) (layer "F.Cu") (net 2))
 (segment (start 45.25 30.050000000000004) (end 45.150000000000006 29.950000000000003) (width 0.2) (layer "B.Cu") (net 4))
 (segment (start 45.150000000000006 29.950000000000003) (end 45.050000000000004 29.950000000000003) (width 0.2) (layer "B.Cu") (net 4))
 (segment (start 45.050000000000004 29.950000000000003) (end 44.95 29.85) (width 0.2) (layer "B.Cu") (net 4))
 (segment (start 44.95 29.85) (end 44.050000000000004 29.85) (width 0.2) (layer "B.Cu") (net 4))
 (segment (start 44.050000000000004 29.85) (end 40.25 26.05) (width 0.2) (layer "B.Cu") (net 4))
 (segment (start 40.25 26.05) (end 40.25 25.25) (width 0.2) (layer "B.Cu") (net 4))
 (segment (start 40.25 25.25) (end 39.550000000000004 24.55) (width 0.2) (layer "B.Cu") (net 4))
 (segment (start 39.550000000000004 24.55) (end 36.45 24.55) (width 0.2) (layer "B.Cu") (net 4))
 (segment (start 36.45 24.55) (end 27.55 15.650000000000002) (width 0.2) (layer "B.Cu") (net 4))
 (segment (start 27.55 15.650000000000002) (end 27.55 15.55) (width 0.2) (layer "B.Cu") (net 4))
 (segment (start 27.55 15.55) (end 27.05 15.05) (width 0.2) (layer "B.Cu") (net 4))
 (segment (start 27.05 15.05) (end 25.450000000000003 15.05) (width 0.2) (layer "B.Cu") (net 4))
 (segment (start 25.450000000000003 15.05) (end 25.450000000000003 16.45) (width 0.2) (layer "B.Cu") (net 4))
 (segment (start 25.450000000000003 16.45) (end 25.650000000000002 16.650000000000002) (width 0.2) (layer "B.Cu") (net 4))
 (segment (start 25.650000000000002 16.650000000000002) (end 25.650000000000002 18.150000000000002) (width 0.2) (layer "B.Cu") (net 4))
 (segment (start 25.650000000000002 18.150000000000002) (end 25.75 18.25) (width 0.2) (layer "B.Cu") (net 4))
 (segment (start 25.75 18.25) (end 25.75 19.75) (width 0.2) (layer "B.Cu") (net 4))
 (segment (start 25.75 19.75) (end 31.25 25.25) (width 0.2) (layer "B.Cu") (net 4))
 (segment (start 31.25 25.25) (end 31.25 28.25) (width 0.2) (layer "B.Cu") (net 4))
 (segment (start 31.25 28.25) (end 31.65 28.650000000000002) (width 0.2) (layer "B.Cu") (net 4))
 (segment (start 31.65 28.650000000000002) (end 31.65 31.35) (width 0.2) (layer "B.Cu") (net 4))
 (segment (start 31.65 31.35) (end 31.25 31.75) (width 0.2) (layer "B.Cu") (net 4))
 (segment (start 31.25 31.75) (end 31.25 34.75) (width 0.2) (layer "B.Cu") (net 4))
 (segment (start 31.25 34.75) (end 25.05 40.95) (width 0.2) (layer "B.Cu") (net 4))
 (segment (start 25.05 40.95) (end 25.05 60.050000000000004) (width 0.2) (layer "B.Cu") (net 4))
 (segment (start 30.050000000000004 45.050000000000004) (end 31.450000000000003 45.050000000000004) (width 0.2) (layer "F.Cu") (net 5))
 (segment (start 31.450000000000003 45.050000000000004) (end 31.65 44.85) (width 0.2) (layer "F.Cu") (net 5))
 (segment (start 31.65 44.85) (end 33.15 44.85) (width 0.2) (layer "F.Cu") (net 5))
 (segment (start 33.15 44.85) (end 33.25 44.75) (width 0.2) (layer "F.Cu") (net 5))
 (segment (start 33.25 44.75) (end 42.45 44.75) (width 0.2) (layer "F.Cu") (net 5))
 (segment (start 42.45 44.75) (end 43.75 43.45) (width 0.2) (layer "F.Cu") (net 5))
 (segment (start 43.75 43.45) (end 43.85 43.45) (width 0.2) (layer "F.Cu") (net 5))
 (segment (start 43.85 43.45) (end 43.95 43.35) (width 0.2) (layer "F.Cu") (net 5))
 (segment (start 43.95 43.35) (end 46.550000000000004 43.35) (width 0.2) (layer "F.Cu") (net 5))
 (segment (start 46.550000000000004 43.35) (end 46.85 43.650000000000006) (width 0.2) (layer "F.Cu") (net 5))
 (segment (start 46.85 43.650000000000006) (end 46.85 49.35) (width 0.2) (layer "F.Cu") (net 5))
 (segment (start 46.85 49.35) (end 50.95 53.45) (width 0.2) (layer "F.Cu") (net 5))
 (segment (start 50.95 53.45) (end 50.95 54.25) (width 0.2) (layer "F.Cu") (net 5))
 (segment (start 50.95 54.25) (end 51.050000000000004 54.35) (width 0.2) (layer "F.Cu") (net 5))
 (segment (start 51.050000000000004 54.35) (end 51.050000000000004 56.95) (width 0.2) (layer "F.Cu") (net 5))
 (segment (start 51.050000000000004 56.95) (end 52.35 58.25) (width 0.2) (layer "F.Cu") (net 5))
 (segment (start 52.35 58.25) (end 52.35 59.85) (width 0.2) (layer "F.Cu") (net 5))
 (segment (start 52.35 59.85) (end 52.550000000000004 60.050000000000004) (width 0.2) (layer "F.Cu") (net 5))
 (segment (start 52.550000000000004 60.050000000000004) (end 52.550000000000004 39.35) (width 0.2) (layer "F.Cu") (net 5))
 (segment (start 52.550000000000004 39.35) (end 52.650000000000006 39.25) (width 0.2) (layer "F.Cu") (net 5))
 (segment (start 52.650000000000006 39.25) (end 52.650000000000006 26.85) (width 0.2) (layer "F.Cu") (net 5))
 (segment (start 52.650000000000006 26.85) (end 52.95 26.55) (width 0.2) (layer "F.Cu") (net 5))
 (segment (start 52.95 26.55) (end 52.95 19.85) (width 0.2) (layer "F.Cu") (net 5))
 (segment (start 52.95 19.85) (end 55.75 17.05) (width 0.2) (layer "F.Cu") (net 5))
 (segment (start 55.75 17.05) (end 55.75 15.150000000000002) (width 0.2) (layer "F.Cu") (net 5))
 (segment (start 55.75 15.150000000000002) (end 55.85 15.05) (width 0.2) (layer "F.Cu") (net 5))
 (segment (start 78.79999995231628 96.55) (end 27.09999990463257 109.02499997615814) (width 0.2) (layer "B.Cu") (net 22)))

